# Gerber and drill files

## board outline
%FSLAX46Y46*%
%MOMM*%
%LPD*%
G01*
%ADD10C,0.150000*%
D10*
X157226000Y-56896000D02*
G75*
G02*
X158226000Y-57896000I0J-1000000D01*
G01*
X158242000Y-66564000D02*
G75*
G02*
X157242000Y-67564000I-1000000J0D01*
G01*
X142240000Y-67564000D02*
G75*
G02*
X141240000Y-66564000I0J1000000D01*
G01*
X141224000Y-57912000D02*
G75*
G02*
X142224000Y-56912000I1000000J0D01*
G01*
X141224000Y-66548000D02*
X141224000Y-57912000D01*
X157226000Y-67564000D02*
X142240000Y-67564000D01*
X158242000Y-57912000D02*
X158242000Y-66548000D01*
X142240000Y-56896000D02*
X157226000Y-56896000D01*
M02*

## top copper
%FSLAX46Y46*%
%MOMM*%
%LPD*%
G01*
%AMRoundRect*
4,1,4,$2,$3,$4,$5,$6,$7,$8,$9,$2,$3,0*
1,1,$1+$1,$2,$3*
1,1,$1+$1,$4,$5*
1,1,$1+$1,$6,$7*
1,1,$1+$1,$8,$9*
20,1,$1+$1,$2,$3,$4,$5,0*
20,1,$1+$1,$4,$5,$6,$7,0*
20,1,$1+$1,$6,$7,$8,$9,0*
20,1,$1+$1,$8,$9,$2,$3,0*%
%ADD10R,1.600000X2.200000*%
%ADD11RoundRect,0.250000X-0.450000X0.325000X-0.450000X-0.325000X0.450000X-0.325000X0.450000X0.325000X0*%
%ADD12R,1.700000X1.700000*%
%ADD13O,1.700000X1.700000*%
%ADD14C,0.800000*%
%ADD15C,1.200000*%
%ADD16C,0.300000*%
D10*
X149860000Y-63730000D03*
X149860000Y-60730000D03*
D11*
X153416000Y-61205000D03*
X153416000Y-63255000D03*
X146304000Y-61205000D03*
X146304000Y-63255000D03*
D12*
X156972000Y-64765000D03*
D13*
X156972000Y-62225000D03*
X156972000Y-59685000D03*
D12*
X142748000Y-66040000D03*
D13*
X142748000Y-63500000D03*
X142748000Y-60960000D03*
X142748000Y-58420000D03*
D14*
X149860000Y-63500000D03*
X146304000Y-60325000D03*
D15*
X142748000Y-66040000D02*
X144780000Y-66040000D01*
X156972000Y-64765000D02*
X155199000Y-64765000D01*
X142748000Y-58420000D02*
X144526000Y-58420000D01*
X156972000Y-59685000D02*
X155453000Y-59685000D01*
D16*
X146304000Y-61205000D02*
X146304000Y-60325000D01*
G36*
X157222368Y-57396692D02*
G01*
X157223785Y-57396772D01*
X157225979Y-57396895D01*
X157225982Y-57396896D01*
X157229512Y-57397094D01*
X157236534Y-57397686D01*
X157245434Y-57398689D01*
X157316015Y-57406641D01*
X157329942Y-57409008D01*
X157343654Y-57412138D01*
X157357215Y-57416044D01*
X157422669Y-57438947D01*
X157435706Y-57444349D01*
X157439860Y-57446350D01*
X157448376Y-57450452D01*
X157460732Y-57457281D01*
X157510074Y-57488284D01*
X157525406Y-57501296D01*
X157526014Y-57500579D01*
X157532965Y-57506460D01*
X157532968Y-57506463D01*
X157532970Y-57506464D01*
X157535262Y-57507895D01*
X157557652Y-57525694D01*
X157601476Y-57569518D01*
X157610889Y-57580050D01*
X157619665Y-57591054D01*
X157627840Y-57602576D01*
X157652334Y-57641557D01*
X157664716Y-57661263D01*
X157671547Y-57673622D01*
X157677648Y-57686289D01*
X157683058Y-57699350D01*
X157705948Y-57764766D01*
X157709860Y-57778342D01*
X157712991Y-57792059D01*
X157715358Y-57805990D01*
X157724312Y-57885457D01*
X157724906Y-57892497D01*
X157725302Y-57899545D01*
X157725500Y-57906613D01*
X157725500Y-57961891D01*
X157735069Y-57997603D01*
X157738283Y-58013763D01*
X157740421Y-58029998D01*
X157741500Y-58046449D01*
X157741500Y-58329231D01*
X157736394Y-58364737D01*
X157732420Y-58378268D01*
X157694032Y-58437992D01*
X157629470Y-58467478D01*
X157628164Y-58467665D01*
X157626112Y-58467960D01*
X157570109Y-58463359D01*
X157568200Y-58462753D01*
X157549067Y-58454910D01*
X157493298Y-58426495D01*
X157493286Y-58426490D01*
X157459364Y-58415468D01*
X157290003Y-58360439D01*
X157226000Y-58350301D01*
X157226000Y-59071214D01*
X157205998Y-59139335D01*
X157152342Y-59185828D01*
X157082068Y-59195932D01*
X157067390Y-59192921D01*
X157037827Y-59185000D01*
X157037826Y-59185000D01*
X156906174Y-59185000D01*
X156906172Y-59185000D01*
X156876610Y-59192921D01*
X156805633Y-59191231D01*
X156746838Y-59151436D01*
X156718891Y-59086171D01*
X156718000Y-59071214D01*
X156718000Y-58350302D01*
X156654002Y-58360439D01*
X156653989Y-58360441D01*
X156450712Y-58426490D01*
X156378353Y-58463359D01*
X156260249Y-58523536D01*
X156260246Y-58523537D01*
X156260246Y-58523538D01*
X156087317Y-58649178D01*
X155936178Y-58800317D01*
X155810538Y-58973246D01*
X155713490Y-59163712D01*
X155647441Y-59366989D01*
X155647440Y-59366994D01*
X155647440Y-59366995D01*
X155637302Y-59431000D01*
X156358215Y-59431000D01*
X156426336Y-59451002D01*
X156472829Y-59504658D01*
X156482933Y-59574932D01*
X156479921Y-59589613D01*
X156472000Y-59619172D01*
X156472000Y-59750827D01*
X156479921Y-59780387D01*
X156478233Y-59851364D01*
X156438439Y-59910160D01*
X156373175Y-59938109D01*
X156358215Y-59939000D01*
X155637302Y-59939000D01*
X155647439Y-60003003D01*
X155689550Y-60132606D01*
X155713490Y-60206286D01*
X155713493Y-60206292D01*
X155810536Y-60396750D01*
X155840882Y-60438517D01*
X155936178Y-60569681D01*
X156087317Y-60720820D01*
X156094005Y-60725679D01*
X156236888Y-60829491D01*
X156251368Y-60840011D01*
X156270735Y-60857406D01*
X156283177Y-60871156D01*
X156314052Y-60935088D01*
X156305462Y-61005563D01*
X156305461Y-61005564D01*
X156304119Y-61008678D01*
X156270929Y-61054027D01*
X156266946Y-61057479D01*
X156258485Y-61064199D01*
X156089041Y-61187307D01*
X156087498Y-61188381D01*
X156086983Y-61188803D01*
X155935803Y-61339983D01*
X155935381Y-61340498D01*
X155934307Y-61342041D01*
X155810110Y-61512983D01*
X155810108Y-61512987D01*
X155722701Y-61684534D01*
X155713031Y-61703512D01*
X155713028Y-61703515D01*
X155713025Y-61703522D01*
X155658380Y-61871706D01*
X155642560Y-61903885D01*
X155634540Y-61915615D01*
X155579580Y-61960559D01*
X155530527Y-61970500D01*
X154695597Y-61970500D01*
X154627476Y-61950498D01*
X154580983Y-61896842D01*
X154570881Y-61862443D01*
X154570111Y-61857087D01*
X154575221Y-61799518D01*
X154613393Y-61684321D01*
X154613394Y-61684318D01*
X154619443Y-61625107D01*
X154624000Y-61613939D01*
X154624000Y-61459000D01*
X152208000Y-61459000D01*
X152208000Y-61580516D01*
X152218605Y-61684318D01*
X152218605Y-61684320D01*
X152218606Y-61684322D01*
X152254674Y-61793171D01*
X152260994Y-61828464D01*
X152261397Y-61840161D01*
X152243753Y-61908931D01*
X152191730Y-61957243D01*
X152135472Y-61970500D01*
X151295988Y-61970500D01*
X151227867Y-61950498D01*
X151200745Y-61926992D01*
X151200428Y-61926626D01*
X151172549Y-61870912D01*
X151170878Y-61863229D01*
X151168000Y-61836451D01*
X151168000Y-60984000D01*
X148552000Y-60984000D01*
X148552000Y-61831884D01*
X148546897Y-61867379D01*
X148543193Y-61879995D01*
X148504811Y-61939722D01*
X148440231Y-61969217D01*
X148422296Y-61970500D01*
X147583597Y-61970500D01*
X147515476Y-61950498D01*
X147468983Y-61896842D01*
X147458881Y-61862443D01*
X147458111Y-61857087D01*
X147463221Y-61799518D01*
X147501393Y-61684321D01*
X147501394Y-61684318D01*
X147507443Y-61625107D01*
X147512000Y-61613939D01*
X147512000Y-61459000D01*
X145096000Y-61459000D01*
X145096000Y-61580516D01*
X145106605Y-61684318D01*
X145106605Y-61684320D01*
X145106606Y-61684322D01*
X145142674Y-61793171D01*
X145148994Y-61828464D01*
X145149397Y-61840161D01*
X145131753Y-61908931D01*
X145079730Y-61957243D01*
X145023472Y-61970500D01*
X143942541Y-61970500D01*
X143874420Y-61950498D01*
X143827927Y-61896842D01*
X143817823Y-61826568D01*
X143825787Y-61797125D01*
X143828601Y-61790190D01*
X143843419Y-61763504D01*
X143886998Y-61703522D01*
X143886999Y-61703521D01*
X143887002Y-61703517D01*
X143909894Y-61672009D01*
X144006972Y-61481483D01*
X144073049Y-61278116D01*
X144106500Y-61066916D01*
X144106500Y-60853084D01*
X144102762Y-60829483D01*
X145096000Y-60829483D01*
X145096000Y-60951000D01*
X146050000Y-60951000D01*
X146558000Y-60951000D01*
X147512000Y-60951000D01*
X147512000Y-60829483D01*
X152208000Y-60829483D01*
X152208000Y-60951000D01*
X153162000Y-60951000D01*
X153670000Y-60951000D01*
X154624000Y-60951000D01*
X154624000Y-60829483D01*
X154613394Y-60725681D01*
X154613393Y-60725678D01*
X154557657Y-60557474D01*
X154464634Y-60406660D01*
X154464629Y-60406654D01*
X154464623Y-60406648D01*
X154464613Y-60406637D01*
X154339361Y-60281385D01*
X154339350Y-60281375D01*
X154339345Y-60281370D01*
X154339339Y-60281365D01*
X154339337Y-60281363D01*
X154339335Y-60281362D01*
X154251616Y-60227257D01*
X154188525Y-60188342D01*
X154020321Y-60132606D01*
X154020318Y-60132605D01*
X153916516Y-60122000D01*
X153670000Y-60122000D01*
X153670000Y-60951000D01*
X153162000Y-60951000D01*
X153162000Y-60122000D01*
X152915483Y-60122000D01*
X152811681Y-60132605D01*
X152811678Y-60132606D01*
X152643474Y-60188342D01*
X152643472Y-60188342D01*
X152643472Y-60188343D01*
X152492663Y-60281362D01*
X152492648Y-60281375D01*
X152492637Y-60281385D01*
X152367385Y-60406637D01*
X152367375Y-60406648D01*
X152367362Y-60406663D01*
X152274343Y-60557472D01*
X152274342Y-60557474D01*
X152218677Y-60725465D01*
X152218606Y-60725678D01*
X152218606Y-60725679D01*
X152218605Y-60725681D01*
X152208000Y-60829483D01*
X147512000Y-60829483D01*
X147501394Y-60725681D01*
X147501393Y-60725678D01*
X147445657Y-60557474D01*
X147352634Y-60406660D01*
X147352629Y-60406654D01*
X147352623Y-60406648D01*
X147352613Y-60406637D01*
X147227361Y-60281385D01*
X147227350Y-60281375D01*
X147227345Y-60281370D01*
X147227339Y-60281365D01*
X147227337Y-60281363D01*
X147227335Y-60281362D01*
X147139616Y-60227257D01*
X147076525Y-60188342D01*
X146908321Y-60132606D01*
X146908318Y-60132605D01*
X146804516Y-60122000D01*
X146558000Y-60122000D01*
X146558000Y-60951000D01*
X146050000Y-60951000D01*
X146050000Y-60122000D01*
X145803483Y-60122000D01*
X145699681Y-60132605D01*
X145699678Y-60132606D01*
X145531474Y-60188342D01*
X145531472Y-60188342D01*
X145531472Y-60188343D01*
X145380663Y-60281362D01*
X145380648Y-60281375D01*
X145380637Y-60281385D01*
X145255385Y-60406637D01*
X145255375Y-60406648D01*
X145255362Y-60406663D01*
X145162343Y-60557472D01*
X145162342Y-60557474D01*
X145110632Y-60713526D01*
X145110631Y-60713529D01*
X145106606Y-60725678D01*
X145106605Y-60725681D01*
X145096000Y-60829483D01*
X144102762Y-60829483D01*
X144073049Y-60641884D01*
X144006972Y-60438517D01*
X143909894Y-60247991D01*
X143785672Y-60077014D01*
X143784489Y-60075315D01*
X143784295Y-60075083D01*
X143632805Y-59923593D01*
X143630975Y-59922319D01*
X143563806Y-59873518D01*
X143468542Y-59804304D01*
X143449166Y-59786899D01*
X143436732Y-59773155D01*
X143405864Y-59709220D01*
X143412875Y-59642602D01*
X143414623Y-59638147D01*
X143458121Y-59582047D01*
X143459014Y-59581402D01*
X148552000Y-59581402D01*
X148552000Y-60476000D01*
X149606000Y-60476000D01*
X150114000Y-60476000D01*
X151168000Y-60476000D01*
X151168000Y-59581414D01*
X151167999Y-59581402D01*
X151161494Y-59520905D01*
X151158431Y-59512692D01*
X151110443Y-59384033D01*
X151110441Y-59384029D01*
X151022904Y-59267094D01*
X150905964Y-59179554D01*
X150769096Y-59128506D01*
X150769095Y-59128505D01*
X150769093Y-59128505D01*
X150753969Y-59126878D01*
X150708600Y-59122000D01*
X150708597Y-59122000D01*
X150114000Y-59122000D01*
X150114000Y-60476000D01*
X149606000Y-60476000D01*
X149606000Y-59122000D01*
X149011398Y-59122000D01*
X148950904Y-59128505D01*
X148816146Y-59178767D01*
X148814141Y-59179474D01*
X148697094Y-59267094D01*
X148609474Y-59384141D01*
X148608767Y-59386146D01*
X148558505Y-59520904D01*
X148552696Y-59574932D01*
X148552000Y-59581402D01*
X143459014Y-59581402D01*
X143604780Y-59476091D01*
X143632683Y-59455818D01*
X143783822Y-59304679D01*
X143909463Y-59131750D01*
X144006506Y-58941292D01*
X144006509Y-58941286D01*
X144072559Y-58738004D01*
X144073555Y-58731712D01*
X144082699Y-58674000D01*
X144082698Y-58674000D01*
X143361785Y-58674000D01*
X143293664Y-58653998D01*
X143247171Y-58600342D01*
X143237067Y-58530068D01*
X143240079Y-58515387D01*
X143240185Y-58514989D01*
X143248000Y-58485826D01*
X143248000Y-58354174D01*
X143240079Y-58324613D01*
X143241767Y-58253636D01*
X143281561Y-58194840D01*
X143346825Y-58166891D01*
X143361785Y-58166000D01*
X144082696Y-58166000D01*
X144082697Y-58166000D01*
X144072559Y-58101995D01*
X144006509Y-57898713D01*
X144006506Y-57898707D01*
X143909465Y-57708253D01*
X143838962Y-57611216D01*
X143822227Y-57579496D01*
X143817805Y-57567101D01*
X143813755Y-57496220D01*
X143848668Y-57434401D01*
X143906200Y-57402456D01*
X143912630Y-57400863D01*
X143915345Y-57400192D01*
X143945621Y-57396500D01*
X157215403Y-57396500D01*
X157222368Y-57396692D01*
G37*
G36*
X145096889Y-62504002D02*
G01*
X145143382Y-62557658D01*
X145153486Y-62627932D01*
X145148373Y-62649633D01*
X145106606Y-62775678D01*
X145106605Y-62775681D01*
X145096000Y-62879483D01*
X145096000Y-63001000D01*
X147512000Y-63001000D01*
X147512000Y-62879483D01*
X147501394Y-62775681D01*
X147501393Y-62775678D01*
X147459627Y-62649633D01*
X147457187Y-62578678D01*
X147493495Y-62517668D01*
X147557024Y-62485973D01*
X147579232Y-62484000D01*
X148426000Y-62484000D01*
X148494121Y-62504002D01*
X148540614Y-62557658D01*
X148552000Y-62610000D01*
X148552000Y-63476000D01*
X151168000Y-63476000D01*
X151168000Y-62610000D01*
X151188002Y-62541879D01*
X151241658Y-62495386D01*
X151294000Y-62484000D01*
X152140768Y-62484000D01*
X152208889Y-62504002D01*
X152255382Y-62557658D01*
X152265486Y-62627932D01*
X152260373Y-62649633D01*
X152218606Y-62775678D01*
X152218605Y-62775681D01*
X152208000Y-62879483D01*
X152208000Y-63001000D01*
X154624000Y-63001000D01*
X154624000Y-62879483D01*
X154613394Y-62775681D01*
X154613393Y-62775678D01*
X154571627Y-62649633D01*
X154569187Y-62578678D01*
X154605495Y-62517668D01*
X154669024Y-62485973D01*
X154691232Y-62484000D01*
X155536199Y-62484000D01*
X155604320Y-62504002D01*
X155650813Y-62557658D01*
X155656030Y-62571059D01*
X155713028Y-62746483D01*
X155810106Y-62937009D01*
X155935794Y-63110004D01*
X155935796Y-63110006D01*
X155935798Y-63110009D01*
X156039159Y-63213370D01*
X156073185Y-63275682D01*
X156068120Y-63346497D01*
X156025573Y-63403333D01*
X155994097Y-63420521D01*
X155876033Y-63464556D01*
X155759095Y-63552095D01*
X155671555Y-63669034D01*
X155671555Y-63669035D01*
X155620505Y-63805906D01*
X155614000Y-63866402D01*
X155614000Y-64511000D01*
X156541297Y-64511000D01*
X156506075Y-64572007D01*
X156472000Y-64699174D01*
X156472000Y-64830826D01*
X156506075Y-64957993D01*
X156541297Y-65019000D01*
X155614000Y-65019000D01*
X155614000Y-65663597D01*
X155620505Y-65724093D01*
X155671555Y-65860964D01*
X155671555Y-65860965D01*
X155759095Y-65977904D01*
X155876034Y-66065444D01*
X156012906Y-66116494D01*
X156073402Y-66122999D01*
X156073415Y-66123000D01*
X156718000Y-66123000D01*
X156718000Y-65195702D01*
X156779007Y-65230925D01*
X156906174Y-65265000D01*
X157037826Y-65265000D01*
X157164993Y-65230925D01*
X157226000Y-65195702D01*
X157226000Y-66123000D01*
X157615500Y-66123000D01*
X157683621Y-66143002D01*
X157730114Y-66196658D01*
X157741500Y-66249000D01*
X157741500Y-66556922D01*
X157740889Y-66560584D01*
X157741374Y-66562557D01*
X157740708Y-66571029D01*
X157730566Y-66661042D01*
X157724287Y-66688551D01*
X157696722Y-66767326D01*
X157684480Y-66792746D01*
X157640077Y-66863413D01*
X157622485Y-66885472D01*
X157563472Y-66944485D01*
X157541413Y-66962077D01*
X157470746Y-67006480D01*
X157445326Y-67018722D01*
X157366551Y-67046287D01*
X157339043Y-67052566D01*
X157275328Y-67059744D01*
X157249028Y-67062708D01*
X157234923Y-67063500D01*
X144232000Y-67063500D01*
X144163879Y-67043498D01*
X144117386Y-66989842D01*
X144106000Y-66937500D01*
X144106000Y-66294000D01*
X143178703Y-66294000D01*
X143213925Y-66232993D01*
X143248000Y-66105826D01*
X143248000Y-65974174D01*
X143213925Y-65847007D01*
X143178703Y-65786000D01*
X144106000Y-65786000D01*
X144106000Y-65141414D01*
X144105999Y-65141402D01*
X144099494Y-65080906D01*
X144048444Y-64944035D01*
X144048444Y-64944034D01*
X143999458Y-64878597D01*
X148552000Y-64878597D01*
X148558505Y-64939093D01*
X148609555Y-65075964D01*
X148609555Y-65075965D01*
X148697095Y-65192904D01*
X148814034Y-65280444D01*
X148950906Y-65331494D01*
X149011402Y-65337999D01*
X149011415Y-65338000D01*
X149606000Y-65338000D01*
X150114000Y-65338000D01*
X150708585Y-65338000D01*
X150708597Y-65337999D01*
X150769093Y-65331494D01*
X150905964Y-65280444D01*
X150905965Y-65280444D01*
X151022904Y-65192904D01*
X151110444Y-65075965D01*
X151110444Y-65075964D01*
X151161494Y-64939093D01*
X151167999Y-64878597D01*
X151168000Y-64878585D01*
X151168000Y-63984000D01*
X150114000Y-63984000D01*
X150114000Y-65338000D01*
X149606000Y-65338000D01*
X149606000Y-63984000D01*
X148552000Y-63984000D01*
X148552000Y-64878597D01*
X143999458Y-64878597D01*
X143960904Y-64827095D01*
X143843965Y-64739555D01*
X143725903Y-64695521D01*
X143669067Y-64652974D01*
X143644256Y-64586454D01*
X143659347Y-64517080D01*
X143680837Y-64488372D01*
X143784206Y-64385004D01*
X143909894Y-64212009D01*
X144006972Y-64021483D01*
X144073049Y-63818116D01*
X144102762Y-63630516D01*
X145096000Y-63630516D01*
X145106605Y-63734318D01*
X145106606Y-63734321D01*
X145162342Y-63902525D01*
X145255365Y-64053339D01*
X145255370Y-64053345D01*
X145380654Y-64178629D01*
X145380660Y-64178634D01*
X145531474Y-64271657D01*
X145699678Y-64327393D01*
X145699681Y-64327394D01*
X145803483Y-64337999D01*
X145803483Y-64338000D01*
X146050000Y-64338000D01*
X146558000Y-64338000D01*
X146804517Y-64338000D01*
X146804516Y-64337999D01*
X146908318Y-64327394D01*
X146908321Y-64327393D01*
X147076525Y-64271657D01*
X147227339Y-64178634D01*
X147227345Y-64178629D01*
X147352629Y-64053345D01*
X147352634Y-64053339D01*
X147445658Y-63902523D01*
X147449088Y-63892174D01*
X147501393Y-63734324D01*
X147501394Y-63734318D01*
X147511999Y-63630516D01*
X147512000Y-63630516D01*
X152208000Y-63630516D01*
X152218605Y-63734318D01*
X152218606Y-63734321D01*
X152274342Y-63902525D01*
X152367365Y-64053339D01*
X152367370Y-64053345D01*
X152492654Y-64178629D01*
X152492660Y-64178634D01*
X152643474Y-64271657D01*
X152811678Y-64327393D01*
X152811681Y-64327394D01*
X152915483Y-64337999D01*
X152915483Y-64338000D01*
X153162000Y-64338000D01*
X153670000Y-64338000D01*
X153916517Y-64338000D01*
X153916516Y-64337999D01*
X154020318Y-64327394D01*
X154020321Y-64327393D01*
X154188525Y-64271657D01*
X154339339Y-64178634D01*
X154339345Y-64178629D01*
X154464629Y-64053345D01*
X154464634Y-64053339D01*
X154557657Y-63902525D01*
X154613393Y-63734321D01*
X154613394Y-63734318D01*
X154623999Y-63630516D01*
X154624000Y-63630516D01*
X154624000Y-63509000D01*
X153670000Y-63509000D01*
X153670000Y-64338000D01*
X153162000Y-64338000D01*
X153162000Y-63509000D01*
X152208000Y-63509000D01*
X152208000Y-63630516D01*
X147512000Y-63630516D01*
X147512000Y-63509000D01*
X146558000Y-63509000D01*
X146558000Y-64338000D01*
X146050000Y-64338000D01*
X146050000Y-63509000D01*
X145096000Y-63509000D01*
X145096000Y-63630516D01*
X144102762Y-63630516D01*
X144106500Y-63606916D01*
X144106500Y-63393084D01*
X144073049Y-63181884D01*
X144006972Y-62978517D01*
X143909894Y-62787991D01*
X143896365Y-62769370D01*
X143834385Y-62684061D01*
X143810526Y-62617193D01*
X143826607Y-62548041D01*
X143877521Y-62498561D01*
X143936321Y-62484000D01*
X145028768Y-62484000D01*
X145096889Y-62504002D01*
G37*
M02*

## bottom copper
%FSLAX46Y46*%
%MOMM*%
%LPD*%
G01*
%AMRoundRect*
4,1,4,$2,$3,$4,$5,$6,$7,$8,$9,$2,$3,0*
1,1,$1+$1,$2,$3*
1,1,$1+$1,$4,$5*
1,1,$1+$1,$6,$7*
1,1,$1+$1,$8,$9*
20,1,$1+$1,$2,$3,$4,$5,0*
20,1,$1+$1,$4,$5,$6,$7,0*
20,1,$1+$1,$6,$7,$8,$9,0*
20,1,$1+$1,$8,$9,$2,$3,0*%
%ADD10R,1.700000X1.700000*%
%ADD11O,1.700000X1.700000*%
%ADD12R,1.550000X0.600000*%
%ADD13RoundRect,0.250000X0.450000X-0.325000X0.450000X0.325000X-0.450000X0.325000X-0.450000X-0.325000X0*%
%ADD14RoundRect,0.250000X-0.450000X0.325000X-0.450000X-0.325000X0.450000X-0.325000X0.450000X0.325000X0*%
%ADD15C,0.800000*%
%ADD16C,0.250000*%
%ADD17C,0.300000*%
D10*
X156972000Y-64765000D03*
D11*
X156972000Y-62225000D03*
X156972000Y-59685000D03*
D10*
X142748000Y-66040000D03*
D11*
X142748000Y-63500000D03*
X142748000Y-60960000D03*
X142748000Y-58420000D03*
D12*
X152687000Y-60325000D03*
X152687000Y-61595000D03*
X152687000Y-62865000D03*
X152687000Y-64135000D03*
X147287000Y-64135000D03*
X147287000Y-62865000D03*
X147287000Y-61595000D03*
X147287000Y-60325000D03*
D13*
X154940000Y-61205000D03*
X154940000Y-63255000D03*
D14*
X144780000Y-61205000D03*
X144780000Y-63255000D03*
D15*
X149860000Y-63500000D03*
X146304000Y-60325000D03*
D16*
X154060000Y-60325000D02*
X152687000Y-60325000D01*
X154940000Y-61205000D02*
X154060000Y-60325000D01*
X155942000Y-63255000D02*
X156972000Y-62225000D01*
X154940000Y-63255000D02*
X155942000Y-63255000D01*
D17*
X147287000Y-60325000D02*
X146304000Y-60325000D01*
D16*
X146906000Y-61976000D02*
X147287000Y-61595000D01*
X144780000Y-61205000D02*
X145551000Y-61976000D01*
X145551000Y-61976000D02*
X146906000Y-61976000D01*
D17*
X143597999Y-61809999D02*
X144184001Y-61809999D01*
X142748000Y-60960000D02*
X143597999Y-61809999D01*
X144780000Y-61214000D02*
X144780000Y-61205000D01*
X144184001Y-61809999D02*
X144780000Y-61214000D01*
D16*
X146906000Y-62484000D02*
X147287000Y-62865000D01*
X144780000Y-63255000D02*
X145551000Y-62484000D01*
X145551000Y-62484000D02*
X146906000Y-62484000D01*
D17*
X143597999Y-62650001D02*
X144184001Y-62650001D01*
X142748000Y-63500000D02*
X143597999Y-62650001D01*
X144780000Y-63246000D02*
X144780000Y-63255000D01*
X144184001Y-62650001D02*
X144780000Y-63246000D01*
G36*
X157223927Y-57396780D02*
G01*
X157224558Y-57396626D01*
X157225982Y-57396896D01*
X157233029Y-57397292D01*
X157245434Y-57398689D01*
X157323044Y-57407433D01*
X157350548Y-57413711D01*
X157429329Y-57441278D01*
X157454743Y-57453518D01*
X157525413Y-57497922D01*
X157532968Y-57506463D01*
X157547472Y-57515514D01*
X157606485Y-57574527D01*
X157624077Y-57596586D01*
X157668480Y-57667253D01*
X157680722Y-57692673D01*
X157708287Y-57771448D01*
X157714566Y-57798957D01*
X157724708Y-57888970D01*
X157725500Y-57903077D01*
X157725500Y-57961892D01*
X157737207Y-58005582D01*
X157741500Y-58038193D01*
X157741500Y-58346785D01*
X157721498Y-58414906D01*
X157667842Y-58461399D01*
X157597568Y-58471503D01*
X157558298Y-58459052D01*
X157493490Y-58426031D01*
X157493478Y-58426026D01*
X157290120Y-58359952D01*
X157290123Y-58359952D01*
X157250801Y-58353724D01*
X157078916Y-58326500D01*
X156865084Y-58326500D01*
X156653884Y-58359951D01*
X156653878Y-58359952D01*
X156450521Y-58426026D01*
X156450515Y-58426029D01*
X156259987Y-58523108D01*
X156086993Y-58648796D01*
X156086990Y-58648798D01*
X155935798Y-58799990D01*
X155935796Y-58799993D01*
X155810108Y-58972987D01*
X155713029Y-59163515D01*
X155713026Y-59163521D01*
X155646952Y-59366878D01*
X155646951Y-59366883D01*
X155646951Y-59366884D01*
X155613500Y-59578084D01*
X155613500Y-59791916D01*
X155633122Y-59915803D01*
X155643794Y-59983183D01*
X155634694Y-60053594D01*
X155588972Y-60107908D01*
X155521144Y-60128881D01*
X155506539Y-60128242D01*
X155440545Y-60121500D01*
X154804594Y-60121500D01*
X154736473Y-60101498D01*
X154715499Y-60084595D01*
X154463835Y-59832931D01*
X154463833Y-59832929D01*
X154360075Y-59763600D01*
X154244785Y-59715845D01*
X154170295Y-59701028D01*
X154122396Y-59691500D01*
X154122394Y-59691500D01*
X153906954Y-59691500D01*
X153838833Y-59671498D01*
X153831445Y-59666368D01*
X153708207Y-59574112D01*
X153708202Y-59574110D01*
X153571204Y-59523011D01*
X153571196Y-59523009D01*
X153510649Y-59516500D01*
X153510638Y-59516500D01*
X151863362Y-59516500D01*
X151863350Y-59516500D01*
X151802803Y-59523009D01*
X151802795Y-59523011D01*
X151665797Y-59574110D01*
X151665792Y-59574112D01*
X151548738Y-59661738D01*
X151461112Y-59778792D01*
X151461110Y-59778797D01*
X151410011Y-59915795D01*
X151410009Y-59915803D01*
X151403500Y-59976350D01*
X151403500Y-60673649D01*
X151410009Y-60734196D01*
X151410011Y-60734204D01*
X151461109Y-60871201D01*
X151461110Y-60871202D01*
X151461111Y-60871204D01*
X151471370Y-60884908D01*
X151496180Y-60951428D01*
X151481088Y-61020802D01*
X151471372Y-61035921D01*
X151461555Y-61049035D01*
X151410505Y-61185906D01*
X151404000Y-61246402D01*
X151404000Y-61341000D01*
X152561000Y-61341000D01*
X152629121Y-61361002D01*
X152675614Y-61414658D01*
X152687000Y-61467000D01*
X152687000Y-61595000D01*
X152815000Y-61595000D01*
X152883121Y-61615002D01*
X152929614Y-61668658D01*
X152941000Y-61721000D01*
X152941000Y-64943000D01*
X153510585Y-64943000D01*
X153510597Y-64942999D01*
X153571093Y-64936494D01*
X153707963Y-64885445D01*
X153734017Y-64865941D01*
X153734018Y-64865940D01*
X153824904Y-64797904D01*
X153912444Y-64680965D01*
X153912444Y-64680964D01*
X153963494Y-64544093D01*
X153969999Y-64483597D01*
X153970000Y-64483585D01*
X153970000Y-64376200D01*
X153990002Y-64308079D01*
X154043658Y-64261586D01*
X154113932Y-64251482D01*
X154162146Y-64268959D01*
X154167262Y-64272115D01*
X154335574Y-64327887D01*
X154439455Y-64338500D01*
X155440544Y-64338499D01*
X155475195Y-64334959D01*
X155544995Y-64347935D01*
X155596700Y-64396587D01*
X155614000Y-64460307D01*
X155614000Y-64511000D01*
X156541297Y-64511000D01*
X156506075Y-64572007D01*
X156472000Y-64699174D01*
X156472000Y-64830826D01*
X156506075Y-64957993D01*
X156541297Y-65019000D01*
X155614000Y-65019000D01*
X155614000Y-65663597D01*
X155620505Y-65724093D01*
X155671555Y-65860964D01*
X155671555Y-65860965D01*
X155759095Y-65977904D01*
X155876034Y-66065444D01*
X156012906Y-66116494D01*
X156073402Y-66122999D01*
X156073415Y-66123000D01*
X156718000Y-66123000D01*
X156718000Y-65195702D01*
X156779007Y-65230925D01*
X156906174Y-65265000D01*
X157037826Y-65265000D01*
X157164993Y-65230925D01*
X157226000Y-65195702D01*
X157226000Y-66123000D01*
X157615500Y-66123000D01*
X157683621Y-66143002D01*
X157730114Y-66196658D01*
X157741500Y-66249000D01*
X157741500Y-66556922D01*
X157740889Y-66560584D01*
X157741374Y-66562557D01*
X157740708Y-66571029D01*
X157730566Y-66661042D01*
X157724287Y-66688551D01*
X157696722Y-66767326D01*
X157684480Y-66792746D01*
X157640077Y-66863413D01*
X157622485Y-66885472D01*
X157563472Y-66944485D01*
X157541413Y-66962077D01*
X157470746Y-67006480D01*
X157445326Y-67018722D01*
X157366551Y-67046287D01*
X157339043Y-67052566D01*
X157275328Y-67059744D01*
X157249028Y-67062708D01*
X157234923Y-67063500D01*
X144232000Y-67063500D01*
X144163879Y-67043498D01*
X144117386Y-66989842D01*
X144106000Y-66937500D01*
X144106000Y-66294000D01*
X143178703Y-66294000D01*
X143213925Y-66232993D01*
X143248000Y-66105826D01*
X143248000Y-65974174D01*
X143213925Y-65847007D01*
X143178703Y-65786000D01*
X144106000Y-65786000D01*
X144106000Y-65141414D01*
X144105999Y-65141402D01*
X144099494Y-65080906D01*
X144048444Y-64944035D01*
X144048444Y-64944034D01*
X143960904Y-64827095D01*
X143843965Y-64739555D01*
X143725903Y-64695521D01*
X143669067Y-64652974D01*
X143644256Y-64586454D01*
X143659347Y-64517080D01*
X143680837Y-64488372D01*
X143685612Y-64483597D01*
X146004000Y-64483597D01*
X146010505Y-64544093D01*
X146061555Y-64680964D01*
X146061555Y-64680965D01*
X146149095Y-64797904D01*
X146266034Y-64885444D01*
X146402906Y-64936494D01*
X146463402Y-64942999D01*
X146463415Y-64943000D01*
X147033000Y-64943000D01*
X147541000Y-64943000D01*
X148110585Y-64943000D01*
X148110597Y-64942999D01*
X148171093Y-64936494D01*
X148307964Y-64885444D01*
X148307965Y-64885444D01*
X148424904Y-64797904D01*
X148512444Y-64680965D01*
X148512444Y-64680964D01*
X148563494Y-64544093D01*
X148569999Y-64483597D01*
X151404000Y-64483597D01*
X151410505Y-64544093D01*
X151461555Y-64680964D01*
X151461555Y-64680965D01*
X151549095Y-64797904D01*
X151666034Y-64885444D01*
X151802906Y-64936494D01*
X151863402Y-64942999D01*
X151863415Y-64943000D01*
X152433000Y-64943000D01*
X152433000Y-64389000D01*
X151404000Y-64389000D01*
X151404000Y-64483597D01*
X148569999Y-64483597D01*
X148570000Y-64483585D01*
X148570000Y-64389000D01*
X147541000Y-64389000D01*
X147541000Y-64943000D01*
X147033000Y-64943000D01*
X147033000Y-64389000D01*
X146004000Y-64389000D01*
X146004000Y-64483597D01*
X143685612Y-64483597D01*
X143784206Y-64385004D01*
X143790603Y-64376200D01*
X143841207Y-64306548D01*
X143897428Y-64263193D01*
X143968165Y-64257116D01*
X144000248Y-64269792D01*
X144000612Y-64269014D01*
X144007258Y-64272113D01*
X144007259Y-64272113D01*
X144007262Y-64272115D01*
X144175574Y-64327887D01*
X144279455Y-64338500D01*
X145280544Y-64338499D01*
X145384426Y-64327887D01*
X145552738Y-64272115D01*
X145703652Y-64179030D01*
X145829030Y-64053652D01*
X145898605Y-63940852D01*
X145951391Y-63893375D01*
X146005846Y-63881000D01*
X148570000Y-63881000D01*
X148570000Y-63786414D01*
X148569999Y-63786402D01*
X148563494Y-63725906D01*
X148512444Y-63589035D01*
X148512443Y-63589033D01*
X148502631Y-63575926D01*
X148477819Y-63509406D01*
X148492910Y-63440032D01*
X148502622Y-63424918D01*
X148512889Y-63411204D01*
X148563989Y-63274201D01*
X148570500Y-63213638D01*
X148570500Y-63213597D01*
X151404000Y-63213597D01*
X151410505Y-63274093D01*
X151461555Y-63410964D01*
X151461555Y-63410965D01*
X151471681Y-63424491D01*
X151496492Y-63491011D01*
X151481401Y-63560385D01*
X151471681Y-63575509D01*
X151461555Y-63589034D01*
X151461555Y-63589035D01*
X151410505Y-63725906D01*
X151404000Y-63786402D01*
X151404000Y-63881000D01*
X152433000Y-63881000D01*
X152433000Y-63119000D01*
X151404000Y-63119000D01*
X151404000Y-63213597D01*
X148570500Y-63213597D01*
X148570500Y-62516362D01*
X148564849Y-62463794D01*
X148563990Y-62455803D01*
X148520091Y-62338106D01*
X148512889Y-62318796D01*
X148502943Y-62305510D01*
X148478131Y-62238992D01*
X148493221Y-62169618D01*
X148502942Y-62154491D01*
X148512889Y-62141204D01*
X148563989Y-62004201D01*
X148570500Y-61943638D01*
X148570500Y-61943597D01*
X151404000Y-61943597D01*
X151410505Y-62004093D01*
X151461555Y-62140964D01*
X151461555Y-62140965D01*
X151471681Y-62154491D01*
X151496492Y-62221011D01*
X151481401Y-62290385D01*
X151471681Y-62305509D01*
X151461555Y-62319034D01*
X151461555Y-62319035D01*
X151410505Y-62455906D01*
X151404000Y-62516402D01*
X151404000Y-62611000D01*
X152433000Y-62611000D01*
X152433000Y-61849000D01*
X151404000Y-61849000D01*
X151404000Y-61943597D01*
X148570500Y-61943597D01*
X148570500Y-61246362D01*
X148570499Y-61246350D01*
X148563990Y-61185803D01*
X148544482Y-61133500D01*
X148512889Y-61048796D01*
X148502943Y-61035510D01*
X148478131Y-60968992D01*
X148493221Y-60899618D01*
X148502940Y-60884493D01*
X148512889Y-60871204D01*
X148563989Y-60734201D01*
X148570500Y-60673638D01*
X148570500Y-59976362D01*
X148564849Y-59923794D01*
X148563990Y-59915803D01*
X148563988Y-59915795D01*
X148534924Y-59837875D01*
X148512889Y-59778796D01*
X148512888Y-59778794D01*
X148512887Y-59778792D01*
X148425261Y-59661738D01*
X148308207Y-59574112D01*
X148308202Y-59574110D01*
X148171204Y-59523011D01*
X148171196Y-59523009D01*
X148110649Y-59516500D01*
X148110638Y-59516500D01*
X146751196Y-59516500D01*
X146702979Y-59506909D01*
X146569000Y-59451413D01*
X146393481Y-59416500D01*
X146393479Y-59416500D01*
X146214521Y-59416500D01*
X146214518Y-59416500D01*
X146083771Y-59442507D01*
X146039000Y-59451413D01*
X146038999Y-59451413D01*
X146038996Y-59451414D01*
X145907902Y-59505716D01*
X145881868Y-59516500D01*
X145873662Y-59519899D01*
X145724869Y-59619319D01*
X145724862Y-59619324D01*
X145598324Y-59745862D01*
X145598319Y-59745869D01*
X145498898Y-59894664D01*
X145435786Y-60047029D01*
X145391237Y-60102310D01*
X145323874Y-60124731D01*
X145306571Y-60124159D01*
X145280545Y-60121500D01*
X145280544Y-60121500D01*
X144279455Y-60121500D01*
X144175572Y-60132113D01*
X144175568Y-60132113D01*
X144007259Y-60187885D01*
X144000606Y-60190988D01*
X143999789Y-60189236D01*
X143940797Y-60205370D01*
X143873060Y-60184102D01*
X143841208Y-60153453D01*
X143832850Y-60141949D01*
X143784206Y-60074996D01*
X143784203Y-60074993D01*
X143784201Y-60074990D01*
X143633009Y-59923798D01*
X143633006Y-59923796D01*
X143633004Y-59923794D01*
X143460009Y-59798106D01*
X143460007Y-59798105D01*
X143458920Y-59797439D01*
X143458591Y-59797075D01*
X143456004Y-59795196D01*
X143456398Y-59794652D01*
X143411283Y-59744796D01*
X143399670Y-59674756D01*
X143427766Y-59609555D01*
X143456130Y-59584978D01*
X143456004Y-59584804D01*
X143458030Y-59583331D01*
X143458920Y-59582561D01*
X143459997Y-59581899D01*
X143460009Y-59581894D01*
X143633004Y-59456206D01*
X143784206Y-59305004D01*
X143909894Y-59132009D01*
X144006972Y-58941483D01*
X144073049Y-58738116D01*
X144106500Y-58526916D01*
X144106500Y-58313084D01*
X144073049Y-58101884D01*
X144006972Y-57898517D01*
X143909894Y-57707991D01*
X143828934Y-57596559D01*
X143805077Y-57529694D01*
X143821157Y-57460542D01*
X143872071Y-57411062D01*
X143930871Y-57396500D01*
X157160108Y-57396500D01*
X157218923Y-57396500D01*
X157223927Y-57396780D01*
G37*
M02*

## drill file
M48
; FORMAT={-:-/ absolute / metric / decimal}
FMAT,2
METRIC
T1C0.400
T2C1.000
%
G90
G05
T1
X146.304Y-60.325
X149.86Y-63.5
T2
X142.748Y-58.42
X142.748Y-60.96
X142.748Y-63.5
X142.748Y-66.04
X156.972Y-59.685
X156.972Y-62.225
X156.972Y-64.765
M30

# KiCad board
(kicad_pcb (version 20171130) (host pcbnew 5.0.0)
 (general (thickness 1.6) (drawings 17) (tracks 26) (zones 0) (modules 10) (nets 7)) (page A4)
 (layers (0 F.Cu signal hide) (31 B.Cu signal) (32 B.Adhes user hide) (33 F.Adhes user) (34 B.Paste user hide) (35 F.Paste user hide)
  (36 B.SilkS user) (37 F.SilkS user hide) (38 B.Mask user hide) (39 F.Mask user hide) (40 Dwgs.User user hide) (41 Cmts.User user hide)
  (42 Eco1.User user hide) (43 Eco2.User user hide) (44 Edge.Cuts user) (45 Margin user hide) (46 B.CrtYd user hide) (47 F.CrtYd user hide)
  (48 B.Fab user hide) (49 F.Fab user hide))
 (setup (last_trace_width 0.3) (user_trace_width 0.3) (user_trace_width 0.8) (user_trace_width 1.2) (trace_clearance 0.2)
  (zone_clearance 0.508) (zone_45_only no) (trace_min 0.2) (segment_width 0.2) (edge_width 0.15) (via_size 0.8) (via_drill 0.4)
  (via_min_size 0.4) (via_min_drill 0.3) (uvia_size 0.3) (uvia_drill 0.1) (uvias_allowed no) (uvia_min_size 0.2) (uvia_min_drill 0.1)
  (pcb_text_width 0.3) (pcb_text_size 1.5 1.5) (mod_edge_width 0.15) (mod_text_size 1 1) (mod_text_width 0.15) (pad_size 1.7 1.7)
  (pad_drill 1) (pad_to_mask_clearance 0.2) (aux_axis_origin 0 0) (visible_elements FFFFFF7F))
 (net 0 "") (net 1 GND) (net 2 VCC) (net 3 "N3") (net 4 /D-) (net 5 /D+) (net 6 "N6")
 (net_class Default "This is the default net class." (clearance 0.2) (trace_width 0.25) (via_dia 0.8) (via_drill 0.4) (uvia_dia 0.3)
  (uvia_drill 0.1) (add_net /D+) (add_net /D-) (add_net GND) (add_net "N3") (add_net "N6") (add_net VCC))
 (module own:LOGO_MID (layer B.Cu) (at 152.146 67.31 180)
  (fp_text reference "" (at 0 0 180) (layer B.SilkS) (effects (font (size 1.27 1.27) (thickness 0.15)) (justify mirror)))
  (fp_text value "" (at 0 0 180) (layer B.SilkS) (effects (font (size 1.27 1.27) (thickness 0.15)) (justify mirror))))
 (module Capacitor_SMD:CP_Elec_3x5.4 (layer F.Cu) (at 149.86 62.23 270)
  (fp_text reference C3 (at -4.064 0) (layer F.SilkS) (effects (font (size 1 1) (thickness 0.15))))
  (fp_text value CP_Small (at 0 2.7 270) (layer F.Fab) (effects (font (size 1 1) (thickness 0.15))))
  (pad 2 smd rect (at 1.5 0 270) (size 2.2 1.6) (layers F.Cu F.Paste F.Mask) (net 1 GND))
  (pad 1 smd rect (at -1.5 0 270) (size 2.2 1.6) (layers F.Cu F.Paste F.Mask) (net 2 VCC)))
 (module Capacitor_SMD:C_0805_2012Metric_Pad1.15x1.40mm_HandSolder (layer F.Cu) (at 153.416 62.23 270)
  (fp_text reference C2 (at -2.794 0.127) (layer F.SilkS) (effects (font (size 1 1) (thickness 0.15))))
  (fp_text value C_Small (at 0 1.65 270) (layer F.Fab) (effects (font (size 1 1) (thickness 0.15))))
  (pad 1 smd roundrect (at -1.025 0 270) (size 1.15 1.4) (layers F.Cu F.Paste F.Mask) (roundrect_rratio 0.217391) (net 2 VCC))
  (pad 2 smd roundrect (at 1.025 0 270) (size 1.15 1.4) (layers F.Cu F.Paste F.Mask) (roundrect_rratio 0.217391) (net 1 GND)))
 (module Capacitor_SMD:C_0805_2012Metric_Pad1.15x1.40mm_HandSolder (layer F.Cu) (at 146.304 62.23 270)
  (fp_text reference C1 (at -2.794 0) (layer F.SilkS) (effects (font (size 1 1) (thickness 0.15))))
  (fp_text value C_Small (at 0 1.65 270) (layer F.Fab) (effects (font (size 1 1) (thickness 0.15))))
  (pad 1 smd roundrect (at -1.025 0 270) (size 1.15 1.4) (layers F.Cu F.Paste F.Mask) (roundrect_rratio 0.217391) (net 2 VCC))
  (pad 2 smd roundrect (at 1.025 0 270) (size 1.15 1.4) (layers F.Cu F.Paste F.Mask) (roundrect_rratio 0.217391) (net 1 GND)))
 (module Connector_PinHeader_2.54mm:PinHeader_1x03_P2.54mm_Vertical (layer F.Cu) (at 156.972 64.765 180)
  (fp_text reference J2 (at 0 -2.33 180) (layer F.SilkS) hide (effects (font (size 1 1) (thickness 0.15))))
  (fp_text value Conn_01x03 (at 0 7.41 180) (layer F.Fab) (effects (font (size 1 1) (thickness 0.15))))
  (pad 1 thru_hole rect (at 0 0 180) (size 1.7 1.7) (drill 1) (layers *.Cu *.Mask) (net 1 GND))
  (pad 2 thru_hole oval (at 0 2.54 180) (size 1.7 1.7) (drill 1) (layers *.Cu *.Mask) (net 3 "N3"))
  (pad 3 thru_hole oval (at 0 5.08 180) (size 1.7 1.7) (drill 1) (layers *.Cu *.Mask) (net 2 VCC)))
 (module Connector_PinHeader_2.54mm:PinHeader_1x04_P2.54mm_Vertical (layer F.Cu) (at 142.748 66.04 180)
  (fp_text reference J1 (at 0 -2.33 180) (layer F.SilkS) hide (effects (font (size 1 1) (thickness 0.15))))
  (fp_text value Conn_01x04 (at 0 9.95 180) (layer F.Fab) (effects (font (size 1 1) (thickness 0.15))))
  (pad 1 thru_hole rect (at 0 0 180) (size 1.7 1.7) (drill 1) (layers *.Cu *.Mask) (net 1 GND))
  (pad 2 thru_hole oval (at 0 2.54 180) (size 1.7 1.7) (drill 1) (layers *.Cu *.Mask) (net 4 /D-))
  (pad 3 thru_hole oval (at 0 5.08 180) (size 1.7 1.7) (drill 1) (layers *.Cu *.Mask) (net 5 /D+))
  (pad 4 thru_hole oval (at 0 7.62 180) (size 1.7 1.7) (drill 1) (layers *.Cu *.Mask) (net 2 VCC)))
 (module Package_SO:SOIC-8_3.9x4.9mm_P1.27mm (layer B.Cu) (at 149.987 62.23 180)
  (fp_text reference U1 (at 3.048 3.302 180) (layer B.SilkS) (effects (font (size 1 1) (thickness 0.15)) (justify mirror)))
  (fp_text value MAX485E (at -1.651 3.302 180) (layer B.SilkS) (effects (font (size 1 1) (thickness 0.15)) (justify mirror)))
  (pad 1 smd rect (at -2.7 1.905 180) (size 1.55 0.6) (layers B.Cu B.Paste B.Mask) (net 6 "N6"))
  (pad 2 smd rect (at -2.7 0.635 180) (size 1.55 0.6) (layers B.Cu B.Paste B.Mask) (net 1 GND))
  (pad 3 smd rect (at -2.7 -0.635 180) (size 1.55 0.6) (layers B.Cu B.Paste B.Mask) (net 1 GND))
  (pad 4 smd rect (at -2.7 -1.905 180) (size 1.55 0.6) (layers B.Cu B.Paste B.Mask) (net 1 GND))
  (pad 5 smd rect (at 2.7 -1.905 180) (size 1.55 0.6) (layers B.Cu B.Paste B.Mask) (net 1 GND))
  (pad 6 smd rect (at 2.7 -0.635 180) (size 1.55 0.6) (layers B.Cu B.Paste B.Mask) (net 4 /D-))
  (pad 7 smd rect (at 2.7 0.635 180) (size 1.55 0.6) (layers B.Cu B.Paste B.Mask) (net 5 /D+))
  (pad 8 smd rect (at 2.7 1.905 180) (size 1.55 0.6) (layers B.Cu B.Paste B.Mask) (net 2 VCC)))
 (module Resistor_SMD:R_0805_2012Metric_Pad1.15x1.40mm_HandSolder (layer B.Cu) (at 154.94 62.23 90)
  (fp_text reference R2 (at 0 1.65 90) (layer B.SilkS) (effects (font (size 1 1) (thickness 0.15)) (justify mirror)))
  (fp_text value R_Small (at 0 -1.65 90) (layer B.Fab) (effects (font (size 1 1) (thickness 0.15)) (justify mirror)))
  (pad 2 smd roundrect (at 1.025 0 90) (size 1.15 1.4) (layers B.Cu B.Paste B.Mask) (roundrect_rratio 0.217391) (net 6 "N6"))
  (pad 1 smd roundrect (at -1.025 0 90) (size 1.15 1.4) (layers B.Cu B.Paste B.Mask) (roundrect_rratio 0.217391) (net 3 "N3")))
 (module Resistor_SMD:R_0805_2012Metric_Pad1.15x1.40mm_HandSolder (layer B.Cu) (at 144.78 62.23 270)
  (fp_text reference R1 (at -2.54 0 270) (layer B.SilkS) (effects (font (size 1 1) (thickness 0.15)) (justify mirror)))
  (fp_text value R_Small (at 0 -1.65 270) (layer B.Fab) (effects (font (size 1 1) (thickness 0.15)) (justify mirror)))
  (pad 1 smd roundrect (at -1.025 0 270) (size 1.15 1.4) (layers B.Cu B.Paste B.Mask) (roundrect_rratio 0.217391) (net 5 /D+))
  (pad 2 smd roundrect (at 1.025 0 270) (size 1.15 1.4) (layers B.Cu B.Paste B.Mask) (roundrect_rratio 0.217391) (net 4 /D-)))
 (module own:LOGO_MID (layer F.Cu) (at 152.146 64.643 180)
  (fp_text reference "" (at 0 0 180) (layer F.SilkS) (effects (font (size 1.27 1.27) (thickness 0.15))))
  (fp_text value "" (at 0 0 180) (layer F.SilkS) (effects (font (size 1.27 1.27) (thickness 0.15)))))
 (gr_arc (start 157.226 57.896) (end 158.226 57.896) (angle -90) (layer Edge.Cuts) (width 0.15))
 (gr_arc (start 157.242 66.564) (end 157.242 67.564) (angle -90) (layer Edge.Cuts) (width 0.15))
 (gr_arc (start 142.24 66.564) (end 141.24 66.564) (angle -90) (layer Edge.Cuts) (width 0.15))
 (gr_arc (start 142.224 57.912) (end 142.224 56.912) (angle -90) (layer Edge.Cuts) (width 0.15))
 (gr_line (start 141.224 66.548) (end 141.224 57.912) (layer Edge.Cuts) (width 0.15))
 (gr_line (start 157.226 67.564) (end 142.24 67.564) (layer Edge.Cuts) (width 0.15))
 (gr_line (start 158.242 57.912) (end 158.242 66.548) (layer Edge.Cuts) (width 0.15))
 (gr_line (start 142.24 56.896) (end 157.226 56.896) (layer Edge.Cuts) (width 0.15))
 (segment (start 154.06 60.325) (end 152.687 60.325) (width 0.25) (layer B.Cu) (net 6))
 (segment (start 154.94 61.205) (end 154.06 60.325) (width 0.25) (layer B.Cu) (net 6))
 (segment (start 155.942 63.255) (end 156.972 62.225) (width 0.25) (layer B.Cu) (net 3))
 (segment (start 154.94 63.255) (end 155.942 63.255) (width 0.25) (layer B.Cu) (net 3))
 (via (at 149.86 63.5) (size 0.8) (drill 0.4) (layers F.Cu B.Cu) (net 1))
 (segment (start 142.748 66.04) (end 144.78 66.04) (width 1.2) (layer F.Cu) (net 1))
 (segment (start 156.972 64.765) (end 155.199 64.765) (width 1.2) (layer F.Cu) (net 1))
 (segment (start 142.748 58.42) (end 144.526 58.42) (width 1.2) (layer F.Cu) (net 2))
 (segment (start 156.972 59.685) (end 155.453 59.685) (width 1.2) (layer F.Cu) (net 2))
 (via (at 146.304 60.325) (size 0.8) (drill 0.4) (layers F.Cu B.Cu) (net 2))
 (segment (start 147.287 60.325) (end 146.304 60.325) (width 0.3) (layer B.Cu) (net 2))
 (segment (start 146.304 61.205) (end 146.304 60.325) (width 0.3) (layer F.Cu) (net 2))
 (segment (start 146.906 61.976) (end 147.287 61.595) (width 0.25) (layer B.Cu) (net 5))
 (segment (start 144.78 61.205) (end 145.551 61.976) (width 0.25) (layer B.Cu) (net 5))
 (segment (start 145.551 61.976) (end 146.906 61.976) (width 0.25) (layer B.Cu) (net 5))
 (segment (start 143.597999 61.809999) (end 144.184001 61.809999) (width 0.3) (layer B.Cu) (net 5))
 (segment (start 142.748 60.96) (end 143.597999 61.809999) (width 0.3) (layer B.Cu) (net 5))
 (segment (start 144.78 61.214) (end 144.78 61.205) (width 0.3) (layer B.Cu) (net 5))
 (segment (start 144.184001 61.809999) (end 144.78 61.214) (width 0.3) (layer B.Cu) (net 5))
 (segment (start 146.906 62.484) (end 147.287 62.865) (width 0.25) (layer B.Cu) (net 4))
 (segment (start 144.78 63.255) (end 145.551 62.484) (width 0.25) (layer B.Cu) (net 4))
 (segment (start 145.551 62.484) (end 146.906 62.484) (width 0.25) (layer B.Cu) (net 4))
 (segment (start 143.597999 62.650001) (end 144.184001 62.650001) (width 0.3) (layer B.Cu) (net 4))
 (segment (start 142.748 63.5) (end 143.597999 62.650001) (width 0.3) (layer B.Cu) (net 4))
 (segment (start 144.78 63.246) (end 144.78 63.255) (width 0.3) (layer B.Cu) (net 4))
 (segment (start 144.184001 62.650001) (end 144.78 63.246) (width 0.3) (layer B.Cu) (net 4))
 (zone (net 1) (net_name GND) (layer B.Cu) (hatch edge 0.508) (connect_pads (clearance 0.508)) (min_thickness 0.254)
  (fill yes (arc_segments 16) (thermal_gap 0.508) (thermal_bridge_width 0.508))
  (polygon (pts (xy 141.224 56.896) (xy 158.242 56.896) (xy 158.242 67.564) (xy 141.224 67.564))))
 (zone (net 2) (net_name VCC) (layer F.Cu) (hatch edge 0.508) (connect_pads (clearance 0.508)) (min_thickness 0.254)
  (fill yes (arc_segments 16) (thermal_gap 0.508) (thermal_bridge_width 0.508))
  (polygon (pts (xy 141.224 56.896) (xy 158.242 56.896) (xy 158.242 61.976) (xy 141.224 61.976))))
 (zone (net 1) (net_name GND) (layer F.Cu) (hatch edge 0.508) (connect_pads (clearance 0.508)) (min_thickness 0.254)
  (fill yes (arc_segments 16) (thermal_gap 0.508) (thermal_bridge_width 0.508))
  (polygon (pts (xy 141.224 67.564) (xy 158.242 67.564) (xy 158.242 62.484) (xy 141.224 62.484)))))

